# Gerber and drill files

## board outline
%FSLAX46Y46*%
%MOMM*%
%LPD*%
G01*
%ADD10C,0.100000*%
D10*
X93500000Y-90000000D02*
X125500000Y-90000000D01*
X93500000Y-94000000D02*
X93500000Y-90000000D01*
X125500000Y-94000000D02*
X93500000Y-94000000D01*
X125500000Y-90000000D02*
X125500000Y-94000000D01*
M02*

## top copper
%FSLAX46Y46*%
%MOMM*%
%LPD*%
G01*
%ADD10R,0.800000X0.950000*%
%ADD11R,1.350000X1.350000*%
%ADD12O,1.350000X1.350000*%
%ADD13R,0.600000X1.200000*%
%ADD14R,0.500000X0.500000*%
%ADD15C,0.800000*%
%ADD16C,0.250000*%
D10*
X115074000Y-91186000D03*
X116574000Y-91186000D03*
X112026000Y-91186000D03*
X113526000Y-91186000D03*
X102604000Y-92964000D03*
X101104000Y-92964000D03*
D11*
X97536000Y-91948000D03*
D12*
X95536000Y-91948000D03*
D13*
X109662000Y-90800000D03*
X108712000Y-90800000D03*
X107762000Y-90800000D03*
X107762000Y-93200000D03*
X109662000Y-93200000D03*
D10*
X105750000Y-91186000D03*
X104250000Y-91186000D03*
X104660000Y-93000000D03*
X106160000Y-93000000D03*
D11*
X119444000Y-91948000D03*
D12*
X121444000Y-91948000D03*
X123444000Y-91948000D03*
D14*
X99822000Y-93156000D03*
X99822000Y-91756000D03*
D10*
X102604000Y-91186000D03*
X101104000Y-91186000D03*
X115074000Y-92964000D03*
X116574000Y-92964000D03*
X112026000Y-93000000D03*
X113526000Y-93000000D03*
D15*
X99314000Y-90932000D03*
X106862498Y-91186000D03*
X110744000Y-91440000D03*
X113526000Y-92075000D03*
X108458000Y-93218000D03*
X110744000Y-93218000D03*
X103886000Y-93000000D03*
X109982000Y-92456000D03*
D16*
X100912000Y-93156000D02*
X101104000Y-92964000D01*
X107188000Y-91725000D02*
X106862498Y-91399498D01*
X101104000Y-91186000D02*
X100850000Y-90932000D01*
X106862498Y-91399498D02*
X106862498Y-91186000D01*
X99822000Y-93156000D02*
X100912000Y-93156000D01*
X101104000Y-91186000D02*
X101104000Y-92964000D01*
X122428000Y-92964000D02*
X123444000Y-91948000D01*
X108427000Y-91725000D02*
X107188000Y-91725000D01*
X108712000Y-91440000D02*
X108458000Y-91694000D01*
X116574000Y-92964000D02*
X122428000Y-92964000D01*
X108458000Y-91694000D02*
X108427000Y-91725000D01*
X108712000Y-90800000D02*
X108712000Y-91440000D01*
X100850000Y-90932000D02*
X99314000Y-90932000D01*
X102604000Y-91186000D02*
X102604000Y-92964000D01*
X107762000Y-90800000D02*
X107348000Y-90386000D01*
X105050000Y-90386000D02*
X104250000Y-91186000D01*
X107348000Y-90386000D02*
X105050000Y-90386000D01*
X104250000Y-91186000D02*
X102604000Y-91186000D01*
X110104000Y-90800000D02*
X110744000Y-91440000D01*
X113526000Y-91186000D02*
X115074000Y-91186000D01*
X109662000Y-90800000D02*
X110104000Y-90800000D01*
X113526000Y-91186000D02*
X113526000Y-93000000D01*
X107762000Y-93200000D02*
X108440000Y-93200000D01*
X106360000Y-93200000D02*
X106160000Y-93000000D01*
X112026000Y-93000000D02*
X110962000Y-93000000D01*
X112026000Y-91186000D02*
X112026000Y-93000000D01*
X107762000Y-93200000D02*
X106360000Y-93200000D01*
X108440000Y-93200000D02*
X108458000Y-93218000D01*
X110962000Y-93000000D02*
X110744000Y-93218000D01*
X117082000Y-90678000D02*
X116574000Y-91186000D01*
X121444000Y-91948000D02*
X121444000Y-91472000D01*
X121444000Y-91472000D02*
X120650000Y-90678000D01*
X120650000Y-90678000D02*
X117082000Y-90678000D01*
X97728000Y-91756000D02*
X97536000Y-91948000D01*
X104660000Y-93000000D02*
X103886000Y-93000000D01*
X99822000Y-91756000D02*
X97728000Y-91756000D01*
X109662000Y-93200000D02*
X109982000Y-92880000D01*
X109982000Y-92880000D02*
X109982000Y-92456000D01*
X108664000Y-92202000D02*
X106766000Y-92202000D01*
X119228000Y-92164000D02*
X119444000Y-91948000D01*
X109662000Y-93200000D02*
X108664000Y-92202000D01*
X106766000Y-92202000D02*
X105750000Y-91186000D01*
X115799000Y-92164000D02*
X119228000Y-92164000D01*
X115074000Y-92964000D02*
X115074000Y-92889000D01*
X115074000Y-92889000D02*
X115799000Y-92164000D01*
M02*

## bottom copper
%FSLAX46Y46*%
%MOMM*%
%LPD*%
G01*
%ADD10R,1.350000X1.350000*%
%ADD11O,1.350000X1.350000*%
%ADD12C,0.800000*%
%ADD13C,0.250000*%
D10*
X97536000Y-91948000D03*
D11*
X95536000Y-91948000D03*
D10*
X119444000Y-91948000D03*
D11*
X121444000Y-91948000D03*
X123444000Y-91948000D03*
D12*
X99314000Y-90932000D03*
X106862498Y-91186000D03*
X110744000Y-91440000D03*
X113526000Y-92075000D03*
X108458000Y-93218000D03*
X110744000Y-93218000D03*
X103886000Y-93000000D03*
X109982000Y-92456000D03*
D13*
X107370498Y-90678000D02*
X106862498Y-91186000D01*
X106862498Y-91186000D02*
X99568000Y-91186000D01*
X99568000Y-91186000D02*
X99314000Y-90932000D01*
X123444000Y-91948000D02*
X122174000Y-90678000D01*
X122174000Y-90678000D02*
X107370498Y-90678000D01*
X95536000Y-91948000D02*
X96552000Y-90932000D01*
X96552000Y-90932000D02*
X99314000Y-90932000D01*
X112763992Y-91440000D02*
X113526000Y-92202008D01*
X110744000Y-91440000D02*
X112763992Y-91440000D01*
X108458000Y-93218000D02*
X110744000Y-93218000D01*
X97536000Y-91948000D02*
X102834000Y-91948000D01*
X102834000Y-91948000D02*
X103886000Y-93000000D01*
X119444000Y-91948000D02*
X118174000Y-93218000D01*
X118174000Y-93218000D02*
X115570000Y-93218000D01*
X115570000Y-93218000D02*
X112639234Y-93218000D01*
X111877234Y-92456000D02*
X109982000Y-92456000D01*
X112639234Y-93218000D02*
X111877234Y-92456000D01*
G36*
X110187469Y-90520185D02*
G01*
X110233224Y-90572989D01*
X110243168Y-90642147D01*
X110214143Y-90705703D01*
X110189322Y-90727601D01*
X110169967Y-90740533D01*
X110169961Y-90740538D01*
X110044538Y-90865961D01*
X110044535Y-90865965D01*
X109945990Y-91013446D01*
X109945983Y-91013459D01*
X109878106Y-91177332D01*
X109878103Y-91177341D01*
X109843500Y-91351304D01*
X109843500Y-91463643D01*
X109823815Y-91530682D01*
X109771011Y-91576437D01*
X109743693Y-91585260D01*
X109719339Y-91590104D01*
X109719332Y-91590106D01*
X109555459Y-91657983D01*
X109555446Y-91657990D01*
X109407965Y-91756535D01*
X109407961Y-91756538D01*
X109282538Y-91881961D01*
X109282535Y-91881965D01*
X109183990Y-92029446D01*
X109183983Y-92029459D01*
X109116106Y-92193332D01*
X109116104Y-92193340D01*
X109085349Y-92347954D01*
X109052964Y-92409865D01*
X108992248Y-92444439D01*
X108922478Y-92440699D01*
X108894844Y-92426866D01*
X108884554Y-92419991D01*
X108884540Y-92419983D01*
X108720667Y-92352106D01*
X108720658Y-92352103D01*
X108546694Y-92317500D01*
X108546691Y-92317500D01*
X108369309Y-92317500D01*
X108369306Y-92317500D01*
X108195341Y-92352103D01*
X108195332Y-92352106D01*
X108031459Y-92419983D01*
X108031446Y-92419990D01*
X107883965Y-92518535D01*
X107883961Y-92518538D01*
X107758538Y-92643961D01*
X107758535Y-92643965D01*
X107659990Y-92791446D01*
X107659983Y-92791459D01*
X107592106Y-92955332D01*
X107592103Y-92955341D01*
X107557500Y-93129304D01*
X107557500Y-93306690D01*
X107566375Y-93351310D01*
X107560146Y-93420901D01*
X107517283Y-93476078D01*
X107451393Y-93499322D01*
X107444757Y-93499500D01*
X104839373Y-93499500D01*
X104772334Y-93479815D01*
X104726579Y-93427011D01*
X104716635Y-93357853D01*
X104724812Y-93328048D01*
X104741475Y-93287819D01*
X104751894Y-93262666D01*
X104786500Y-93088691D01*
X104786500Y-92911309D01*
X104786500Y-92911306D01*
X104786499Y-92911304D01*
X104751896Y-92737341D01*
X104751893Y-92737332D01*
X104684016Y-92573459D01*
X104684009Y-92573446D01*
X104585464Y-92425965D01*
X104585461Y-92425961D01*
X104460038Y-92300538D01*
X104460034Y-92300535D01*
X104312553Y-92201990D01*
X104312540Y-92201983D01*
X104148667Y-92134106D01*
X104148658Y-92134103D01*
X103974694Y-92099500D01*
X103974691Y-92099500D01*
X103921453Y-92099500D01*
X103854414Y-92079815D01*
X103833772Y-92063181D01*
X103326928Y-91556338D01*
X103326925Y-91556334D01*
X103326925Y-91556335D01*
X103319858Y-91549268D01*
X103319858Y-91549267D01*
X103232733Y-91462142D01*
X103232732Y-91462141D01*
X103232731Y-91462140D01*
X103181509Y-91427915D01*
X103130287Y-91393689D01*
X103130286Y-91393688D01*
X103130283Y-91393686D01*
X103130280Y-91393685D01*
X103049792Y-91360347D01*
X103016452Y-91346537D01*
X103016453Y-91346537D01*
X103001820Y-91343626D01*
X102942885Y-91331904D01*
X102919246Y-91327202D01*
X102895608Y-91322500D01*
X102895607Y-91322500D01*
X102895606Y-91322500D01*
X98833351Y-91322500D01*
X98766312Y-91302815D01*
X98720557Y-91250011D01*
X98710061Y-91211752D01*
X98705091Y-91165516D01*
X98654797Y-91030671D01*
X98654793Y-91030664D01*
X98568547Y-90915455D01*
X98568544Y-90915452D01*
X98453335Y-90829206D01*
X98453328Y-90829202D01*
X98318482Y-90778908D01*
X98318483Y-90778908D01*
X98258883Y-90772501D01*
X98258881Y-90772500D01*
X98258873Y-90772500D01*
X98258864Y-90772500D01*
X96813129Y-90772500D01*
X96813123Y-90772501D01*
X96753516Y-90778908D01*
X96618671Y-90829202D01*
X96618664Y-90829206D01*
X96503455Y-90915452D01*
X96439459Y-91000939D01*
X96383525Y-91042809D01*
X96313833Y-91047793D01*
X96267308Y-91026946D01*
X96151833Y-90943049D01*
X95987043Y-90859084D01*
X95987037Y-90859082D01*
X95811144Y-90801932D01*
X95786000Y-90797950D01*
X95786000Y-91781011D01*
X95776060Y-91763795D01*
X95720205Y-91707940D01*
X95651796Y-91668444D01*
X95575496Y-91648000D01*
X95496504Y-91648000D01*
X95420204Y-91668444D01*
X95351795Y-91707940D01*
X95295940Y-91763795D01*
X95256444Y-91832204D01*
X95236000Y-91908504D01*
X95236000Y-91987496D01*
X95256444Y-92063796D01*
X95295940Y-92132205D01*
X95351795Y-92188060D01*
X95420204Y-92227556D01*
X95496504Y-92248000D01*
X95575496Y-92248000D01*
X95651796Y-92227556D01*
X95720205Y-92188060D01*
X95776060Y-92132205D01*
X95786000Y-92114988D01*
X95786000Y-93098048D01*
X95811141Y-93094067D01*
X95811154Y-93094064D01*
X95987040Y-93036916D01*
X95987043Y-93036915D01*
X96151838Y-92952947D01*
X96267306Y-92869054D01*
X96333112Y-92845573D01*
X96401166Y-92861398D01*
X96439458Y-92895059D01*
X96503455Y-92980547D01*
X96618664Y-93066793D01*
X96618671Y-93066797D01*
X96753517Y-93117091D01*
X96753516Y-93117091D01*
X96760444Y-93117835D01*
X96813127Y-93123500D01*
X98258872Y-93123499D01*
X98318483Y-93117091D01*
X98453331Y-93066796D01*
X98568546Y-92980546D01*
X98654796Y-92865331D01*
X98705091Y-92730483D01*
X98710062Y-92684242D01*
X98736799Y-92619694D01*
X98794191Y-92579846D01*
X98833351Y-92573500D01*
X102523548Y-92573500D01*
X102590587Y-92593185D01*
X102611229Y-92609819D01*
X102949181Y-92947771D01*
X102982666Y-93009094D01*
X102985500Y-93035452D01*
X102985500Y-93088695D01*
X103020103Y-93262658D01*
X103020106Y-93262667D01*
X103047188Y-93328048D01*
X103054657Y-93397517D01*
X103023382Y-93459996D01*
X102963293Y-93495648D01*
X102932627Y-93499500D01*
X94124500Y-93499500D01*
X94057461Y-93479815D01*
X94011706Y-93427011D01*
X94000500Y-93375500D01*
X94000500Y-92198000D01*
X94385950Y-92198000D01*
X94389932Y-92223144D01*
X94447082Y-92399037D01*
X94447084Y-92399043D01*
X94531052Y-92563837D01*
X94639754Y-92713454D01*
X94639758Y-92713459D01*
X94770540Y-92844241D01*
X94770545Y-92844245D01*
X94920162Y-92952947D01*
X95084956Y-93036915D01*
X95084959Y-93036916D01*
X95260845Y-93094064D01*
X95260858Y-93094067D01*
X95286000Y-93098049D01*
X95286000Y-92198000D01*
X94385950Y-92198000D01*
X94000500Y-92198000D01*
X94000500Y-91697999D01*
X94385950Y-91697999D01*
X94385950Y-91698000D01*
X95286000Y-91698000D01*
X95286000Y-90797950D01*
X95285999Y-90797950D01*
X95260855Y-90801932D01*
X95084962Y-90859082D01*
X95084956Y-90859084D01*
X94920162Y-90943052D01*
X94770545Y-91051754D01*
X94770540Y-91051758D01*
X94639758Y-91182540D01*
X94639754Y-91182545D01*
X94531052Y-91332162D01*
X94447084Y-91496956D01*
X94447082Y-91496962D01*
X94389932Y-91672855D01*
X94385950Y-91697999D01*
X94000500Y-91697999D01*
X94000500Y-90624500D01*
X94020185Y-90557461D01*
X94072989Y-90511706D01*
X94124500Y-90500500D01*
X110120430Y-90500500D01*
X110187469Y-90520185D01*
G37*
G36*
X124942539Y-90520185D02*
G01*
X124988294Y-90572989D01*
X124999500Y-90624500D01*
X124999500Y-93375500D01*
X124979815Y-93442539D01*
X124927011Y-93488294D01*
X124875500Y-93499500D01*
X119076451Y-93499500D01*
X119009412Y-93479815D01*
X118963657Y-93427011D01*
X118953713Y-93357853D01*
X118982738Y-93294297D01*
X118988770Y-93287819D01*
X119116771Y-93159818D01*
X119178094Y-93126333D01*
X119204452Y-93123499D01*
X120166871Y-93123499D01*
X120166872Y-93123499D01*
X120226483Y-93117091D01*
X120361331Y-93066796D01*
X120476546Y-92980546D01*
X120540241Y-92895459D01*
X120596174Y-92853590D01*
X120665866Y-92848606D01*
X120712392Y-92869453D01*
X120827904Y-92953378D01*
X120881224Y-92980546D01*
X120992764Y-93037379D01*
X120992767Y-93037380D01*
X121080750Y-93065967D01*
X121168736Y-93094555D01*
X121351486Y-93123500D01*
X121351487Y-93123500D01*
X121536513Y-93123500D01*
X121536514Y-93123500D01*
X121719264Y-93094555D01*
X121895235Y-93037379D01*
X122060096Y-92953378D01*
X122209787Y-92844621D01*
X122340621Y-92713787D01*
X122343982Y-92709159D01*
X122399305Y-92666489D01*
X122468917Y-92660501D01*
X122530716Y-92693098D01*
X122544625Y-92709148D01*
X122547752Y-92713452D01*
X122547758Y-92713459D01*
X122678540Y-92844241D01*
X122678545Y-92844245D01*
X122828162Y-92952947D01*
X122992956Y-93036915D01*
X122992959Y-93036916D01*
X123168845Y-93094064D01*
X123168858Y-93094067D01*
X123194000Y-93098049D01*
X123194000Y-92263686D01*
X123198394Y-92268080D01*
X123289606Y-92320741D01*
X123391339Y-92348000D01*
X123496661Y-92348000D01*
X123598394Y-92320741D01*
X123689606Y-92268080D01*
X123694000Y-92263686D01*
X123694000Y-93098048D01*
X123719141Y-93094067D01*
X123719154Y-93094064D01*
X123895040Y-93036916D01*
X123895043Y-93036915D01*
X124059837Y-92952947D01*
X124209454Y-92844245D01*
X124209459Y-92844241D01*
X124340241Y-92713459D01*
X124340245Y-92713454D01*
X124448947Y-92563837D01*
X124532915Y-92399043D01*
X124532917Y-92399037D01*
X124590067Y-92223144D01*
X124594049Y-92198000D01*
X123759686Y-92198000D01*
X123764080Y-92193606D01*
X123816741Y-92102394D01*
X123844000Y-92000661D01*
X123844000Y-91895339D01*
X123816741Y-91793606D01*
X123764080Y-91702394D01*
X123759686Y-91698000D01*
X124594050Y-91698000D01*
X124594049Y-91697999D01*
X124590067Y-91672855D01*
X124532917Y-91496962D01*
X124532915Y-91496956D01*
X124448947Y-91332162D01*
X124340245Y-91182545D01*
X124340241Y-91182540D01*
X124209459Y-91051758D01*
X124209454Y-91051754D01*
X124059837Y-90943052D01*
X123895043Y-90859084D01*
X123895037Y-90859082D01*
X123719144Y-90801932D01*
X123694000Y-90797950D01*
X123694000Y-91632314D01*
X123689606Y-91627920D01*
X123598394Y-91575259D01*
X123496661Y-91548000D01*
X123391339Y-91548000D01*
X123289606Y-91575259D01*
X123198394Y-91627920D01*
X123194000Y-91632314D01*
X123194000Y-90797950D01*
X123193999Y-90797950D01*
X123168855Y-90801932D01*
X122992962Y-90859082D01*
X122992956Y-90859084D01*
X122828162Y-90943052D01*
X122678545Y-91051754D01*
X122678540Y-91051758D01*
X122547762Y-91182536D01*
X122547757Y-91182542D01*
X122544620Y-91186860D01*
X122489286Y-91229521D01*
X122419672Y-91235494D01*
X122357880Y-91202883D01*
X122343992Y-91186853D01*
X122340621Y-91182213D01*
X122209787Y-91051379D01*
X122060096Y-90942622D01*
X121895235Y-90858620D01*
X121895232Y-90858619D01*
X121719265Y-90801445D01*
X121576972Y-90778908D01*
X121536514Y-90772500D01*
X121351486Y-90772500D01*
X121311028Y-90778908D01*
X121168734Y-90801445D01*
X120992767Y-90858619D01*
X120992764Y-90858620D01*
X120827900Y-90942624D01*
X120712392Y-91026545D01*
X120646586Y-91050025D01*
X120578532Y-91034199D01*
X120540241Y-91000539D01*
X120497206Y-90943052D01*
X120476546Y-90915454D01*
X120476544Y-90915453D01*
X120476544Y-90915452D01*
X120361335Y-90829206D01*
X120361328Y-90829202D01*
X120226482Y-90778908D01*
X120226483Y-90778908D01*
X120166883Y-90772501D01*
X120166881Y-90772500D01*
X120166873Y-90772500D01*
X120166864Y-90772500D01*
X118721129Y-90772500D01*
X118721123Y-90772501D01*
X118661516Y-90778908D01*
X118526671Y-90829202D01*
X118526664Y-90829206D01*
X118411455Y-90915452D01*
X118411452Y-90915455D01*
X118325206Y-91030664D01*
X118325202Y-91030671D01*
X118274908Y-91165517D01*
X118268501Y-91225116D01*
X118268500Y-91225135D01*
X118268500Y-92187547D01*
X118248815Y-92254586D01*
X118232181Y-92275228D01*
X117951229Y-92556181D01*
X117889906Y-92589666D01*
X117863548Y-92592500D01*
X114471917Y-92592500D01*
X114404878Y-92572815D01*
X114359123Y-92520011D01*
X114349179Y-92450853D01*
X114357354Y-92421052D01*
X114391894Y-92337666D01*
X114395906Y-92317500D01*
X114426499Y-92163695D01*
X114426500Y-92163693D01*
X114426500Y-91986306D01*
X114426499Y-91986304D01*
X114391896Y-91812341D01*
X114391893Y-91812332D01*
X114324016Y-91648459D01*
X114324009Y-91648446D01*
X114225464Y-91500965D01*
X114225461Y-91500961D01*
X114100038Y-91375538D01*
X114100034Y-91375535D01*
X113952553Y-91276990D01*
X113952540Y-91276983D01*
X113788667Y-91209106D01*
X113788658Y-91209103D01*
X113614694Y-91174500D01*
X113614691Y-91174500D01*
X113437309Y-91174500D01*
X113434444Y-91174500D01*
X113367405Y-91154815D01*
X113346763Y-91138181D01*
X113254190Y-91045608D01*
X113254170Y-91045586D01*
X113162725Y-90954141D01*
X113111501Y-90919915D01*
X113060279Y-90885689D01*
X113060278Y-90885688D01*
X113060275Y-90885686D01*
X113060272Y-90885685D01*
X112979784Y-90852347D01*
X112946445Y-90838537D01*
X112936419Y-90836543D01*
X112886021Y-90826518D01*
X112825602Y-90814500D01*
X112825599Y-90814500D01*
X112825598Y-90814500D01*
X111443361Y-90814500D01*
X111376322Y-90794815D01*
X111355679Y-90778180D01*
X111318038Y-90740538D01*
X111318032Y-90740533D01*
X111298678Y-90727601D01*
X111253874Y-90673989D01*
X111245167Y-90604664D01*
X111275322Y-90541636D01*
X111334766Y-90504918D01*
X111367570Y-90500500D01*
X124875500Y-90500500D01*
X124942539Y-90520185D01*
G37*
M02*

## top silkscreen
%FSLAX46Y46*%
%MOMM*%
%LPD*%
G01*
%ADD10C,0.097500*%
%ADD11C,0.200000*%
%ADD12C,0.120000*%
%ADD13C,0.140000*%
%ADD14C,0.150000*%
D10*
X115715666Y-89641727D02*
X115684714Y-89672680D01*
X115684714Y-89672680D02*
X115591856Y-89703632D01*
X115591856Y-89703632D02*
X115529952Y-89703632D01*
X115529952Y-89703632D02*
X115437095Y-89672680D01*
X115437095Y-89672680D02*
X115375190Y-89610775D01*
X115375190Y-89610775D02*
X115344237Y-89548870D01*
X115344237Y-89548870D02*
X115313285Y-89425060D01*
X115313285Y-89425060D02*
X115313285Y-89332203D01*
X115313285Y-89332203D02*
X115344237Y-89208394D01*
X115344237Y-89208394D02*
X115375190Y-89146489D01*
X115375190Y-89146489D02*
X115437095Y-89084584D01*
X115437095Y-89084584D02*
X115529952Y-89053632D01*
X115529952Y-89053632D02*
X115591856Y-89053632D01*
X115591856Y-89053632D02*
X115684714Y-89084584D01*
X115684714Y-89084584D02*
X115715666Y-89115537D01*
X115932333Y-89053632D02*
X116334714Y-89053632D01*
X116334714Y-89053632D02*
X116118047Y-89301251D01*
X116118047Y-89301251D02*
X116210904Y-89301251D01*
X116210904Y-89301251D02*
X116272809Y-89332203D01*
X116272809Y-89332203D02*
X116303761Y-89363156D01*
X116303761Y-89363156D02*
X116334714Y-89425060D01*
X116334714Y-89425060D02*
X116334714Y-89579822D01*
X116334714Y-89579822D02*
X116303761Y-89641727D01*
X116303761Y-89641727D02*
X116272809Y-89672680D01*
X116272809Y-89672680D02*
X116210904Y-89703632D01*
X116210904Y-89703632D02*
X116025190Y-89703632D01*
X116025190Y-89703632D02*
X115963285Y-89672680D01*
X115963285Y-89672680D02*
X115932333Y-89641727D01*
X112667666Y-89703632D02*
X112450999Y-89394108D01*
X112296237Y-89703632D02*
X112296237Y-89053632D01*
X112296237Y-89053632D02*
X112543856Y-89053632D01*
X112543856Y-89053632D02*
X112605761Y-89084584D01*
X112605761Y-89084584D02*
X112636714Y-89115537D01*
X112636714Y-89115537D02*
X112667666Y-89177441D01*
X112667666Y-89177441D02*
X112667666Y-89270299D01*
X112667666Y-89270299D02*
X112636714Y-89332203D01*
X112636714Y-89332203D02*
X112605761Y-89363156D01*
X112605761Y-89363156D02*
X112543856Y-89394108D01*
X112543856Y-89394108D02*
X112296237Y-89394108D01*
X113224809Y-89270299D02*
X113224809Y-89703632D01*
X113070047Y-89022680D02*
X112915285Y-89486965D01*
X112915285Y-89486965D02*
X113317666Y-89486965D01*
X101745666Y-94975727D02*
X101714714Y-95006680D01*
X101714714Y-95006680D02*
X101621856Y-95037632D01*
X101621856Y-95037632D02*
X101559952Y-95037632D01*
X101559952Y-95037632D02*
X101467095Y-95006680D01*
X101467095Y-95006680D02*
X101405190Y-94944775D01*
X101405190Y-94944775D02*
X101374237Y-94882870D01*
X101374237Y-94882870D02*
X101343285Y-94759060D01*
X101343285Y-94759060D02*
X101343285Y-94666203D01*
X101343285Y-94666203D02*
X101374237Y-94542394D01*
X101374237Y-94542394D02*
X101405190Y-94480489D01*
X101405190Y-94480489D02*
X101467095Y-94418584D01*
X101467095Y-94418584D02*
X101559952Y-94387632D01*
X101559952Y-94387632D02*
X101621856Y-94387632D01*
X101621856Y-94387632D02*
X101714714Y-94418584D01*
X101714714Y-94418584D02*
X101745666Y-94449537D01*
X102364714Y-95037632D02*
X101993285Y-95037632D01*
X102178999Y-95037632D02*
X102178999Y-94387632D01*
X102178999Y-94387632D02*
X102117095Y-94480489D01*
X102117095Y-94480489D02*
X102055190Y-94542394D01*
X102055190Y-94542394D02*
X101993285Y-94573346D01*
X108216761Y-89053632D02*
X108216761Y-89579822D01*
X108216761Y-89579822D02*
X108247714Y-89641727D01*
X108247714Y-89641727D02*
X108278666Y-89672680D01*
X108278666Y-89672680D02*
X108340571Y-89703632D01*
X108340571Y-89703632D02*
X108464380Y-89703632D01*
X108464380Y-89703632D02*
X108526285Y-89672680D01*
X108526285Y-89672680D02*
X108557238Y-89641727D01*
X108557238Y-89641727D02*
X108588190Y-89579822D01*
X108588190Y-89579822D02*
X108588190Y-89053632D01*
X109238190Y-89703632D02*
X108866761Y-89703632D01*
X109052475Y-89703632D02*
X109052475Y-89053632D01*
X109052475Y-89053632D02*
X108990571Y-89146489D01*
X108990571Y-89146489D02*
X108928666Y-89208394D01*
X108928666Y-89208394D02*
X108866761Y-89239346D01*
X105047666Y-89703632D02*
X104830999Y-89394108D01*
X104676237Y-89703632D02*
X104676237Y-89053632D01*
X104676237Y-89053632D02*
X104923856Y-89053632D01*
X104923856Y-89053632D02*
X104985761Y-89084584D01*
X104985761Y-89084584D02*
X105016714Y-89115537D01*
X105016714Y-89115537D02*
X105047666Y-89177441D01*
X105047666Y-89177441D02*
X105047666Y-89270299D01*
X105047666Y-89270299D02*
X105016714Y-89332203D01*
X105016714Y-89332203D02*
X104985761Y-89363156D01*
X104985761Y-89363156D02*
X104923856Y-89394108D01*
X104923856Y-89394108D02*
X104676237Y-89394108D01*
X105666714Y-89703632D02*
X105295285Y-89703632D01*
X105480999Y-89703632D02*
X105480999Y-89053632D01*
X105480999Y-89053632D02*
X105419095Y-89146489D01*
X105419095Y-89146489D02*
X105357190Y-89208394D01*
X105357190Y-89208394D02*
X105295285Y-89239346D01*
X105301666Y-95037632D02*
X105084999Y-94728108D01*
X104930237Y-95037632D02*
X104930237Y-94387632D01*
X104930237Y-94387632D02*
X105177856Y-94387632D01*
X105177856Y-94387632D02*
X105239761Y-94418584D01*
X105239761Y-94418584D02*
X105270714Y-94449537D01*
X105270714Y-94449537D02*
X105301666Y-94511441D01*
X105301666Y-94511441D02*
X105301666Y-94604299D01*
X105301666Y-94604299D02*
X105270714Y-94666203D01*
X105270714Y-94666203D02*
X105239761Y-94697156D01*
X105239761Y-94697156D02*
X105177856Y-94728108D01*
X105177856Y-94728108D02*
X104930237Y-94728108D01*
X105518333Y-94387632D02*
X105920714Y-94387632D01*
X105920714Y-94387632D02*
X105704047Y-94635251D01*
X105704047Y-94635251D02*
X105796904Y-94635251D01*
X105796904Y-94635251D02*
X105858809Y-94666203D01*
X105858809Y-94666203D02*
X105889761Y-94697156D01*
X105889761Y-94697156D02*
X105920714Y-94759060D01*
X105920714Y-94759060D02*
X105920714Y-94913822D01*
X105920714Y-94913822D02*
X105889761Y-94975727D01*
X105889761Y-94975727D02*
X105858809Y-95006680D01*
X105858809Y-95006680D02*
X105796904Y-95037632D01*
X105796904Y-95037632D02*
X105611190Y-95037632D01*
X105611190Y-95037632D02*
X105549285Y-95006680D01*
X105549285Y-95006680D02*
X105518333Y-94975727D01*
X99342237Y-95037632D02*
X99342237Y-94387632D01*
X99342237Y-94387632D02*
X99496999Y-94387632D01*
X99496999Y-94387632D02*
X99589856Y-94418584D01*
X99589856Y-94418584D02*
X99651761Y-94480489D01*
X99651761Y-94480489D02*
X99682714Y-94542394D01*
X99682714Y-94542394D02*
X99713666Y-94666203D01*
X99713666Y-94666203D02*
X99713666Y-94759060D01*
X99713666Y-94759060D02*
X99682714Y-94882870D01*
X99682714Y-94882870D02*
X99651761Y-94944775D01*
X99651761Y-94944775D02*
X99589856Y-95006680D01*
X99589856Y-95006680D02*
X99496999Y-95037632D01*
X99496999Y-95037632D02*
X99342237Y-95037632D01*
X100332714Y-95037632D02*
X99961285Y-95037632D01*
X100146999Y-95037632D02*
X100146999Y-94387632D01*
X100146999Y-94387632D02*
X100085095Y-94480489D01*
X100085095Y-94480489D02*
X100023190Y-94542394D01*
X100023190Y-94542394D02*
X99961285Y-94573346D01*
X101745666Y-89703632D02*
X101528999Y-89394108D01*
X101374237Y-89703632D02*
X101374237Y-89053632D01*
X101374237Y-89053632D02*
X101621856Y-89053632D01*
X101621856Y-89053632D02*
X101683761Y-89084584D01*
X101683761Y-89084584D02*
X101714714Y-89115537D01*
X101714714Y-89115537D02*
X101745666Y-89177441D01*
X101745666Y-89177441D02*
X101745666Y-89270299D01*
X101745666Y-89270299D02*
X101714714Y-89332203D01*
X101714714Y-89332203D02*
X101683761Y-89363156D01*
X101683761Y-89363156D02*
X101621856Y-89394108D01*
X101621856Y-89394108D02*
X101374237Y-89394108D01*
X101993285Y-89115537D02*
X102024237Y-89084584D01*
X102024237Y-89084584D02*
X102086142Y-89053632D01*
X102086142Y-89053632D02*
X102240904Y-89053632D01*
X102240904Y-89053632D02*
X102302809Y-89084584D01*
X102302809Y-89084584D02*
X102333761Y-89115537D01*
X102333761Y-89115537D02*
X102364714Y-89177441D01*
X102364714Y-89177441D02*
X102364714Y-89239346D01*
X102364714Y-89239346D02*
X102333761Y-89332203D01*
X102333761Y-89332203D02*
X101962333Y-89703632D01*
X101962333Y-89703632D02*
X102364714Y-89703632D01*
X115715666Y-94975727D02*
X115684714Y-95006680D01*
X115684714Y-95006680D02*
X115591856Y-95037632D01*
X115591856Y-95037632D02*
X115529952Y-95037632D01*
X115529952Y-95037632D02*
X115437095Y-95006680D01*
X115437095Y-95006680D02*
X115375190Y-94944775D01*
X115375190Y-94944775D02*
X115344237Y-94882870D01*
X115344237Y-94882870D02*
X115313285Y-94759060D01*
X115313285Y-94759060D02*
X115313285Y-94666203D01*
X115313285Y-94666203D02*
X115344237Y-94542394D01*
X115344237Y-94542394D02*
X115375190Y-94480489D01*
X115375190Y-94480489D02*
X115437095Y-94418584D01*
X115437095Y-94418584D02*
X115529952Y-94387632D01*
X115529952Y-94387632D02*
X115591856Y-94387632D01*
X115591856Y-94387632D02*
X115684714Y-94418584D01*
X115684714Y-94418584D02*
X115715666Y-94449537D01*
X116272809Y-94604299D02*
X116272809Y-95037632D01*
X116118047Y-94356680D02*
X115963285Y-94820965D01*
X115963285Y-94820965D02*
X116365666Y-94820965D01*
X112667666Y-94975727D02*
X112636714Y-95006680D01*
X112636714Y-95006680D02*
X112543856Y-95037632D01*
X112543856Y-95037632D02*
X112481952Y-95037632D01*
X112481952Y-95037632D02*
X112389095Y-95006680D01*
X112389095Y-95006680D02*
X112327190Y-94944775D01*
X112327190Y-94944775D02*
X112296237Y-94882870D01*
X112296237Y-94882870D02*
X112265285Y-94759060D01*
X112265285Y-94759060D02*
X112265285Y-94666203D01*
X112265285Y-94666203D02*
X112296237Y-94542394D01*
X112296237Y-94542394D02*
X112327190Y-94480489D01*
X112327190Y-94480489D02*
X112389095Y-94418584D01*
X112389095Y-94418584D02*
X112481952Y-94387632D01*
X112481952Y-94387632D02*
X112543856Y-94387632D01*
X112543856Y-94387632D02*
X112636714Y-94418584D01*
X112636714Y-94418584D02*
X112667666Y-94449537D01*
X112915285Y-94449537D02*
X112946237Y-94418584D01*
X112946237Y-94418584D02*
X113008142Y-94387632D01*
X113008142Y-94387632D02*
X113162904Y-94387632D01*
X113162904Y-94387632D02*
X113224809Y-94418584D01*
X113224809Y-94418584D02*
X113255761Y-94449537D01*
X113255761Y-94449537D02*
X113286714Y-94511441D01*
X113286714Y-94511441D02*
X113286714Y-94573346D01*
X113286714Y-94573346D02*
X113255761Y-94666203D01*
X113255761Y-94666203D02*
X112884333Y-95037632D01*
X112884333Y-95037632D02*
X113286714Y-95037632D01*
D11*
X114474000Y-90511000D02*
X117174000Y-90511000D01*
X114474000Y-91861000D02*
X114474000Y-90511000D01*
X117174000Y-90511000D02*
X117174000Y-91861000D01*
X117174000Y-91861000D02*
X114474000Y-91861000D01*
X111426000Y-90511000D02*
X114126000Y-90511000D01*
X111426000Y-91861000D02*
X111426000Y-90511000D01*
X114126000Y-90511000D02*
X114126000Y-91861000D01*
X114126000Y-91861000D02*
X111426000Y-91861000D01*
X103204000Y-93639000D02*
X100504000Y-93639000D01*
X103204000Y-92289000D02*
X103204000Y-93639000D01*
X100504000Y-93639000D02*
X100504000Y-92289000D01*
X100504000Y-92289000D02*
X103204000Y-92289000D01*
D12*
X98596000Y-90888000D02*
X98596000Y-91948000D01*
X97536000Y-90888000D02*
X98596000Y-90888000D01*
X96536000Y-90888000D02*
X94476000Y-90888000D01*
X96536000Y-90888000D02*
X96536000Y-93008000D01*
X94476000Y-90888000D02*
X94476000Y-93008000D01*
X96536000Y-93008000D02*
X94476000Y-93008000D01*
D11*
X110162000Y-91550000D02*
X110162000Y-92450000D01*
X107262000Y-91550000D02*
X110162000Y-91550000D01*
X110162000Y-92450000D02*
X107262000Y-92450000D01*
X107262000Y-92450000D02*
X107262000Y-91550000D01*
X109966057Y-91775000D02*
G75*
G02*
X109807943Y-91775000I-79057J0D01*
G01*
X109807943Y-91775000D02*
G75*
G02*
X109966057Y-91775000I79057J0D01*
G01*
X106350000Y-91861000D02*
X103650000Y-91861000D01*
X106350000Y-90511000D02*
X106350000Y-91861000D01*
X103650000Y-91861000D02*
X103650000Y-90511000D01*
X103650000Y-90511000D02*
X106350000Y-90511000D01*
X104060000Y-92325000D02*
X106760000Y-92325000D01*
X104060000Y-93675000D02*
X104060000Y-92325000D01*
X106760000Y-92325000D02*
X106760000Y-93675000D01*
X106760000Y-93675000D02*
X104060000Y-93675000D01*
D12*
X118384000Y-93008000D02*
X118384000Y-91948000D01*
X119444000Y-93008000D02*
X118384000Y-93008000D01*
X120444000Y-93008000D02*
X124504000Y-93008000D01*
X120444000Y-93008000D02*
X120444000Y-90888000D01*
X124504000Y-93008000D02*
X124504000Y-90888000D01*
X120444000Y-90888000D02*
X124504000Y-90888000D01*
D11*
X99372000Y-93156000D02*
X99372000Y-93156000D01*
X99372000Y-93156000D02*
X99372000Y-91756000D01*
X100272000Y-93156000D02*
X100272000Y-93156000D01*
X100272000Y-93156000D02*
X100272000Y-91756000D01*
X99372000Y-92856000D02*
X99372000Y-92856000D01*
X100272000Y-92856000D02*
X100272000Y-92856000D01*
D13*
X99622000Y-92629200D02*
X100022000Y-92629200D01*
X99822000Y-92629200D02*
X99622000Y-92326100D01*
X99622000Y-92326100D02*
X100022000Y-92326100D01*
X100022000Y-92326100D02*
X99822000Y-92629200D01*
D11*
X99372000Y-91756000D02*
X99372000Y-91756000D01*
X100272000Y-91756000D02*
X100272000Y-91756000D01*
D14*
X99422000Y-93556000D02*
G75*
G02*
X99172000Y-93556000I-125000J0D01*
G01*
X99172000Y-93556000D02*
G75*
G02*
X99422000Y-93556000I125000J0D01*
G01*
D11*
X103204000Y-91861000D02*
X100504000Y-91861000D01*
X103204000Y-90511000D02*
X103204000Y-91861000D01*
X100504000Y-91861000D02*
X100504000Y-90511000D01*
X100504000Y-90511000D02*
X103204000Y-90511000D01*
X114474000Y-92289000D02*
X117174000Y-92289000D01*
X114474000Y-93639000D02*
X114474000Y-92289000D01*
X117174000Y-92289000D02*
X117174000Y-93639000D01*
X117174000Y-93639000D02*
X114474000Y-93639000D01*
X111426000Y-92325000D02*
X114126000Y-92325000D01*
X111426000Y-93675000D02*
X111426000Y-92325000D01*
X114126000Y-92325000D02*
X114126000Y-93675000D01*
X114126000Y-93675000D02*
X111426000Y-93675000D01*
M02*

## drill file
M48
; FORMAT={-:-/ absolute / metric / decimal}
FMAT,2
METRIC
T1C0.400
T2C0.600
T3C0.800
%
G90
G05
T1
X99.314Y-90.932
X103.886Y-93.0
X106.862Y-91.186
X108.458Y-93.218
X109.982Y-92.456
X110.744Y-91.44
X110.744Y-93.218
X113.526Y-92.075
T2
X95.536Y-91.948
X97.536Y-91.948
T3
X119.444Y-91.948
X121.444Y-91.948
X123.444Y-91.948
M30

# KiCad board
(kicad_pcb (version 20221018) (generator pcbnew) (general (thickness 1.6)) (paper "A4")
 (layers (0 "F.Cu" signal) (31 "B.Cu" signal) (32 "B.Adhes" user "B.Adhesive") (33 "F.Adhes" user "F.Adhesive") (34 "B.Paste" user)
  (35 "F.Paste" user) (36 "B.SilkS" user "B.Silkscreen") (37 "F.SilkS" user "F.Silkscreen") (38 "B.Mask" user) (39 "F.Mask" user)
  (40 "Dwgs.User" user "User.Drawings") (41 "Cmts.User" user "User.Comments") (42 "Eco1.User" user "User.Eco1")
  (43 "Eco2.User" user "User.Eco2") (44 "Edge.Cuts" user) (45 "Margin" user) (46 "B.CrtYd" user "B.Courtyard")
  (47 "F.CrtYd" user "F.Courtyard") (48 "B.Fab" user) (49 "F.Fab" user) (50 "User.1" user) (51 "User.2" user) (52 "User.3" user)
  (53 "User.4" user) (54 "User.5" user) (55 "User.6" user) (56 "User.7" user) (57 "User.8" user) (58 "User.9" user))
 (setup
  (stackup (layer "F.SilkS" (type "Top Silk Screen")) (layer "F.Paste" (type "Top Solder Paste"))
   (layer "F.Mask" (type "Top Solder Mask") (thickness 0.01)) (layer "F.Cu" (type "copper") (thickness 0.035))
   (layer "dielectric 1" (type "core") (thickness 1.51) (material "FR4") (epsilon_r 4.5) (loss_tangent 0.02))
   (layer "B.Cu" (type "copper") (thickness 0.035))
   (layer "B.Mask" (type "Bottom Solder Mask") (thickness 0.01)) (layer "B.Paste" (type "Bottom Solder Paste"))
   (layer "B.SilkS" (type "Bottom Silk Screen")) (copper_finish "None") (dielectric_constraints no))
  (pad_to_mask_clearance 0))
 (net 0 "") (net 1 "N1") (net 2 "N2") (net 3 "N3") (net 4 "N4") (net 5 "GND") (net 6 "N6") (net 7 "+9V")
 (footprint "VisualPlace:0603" (layer "F.Cu") (at 115.824 91.186)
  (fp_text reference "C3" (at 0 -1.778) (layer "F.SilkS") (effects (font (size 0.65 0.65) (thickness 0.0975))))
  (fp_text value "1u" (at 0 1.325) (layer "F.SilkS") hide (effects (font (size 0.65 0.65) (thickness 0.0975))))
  (fp_line (start -1.35 -0.675) (end 1.35 -0.675) (stroke (width 0.2) (type solid)) (layer "F.SilkS"))
  (fp_line (start -1.35 0.675) (end -1.35 -0.675) (stroke (width 0.2) (type solid)) (layer "F.SilkS"))
  (fp_line (start 1.35 -0.675) (end 1.35 0.675) (stroke (width 0.2) (type solid)) (layer "F.SilkS"))
  (fp_line (start 1.35 0.675) (end -1.35 0.675) (stroke (width 0.2) (type solid)) (layer "F.SilkS"))
  (pad "1" smd rect (at -0.75 0) (size 0.8 0.95) (layers "F.Cu" "F.Paste" "F.Mask") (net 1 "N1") (thermal_bridge_angle 45))
  (pad "2" smd rect (at 0.75 0) (size 0.8 0.95) (layers "F.Cu" "F.Paste" "F.Mask") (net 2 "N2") (thermal_bridge_angle 45)))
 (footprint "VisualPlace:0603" (layer "F.Cu") (at 112.776 91.186)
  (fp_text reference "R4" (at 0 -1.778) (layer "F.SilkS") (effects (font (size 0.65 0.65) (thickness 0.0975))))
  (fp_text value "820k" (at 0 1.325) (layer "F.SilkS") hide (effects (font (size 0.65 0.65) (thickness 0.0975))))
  (fp_line (start -1.35 -0.675) (end 1.35 -0.675) (stroke (width 0.2) (type solid)) (layer "F.SilkS"))
  (fp_line (start -1.35 0.675) (end -1.35 -0.675) (stroke (width 0.2) (type solid)) (layer "F.SilkS"))
  (fp_line (start 1.35 -0.675) (end 1.35 0.675) (stroke (width 0.2) (type solid)) (layer "F.SilkS"))
  (fp_line (start 1.35 0.675) (end -1.35 0.675) (stroke (width 0.2) (type solid)) (layer "F.SilkS"))
  (pad "1" smd rect (at -0.75 0) (size 0.8 0.95) (layers "F.Cu" "F.Paste" "F.Mask") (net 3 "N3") (thermal_bridge_angle 45))
  (pad "2" smd rect (at 0.75 0) (size 0.8 0.95) (layers "F.Cu" "F.Paste" "F.Mask") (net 1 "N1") (thermal_bridge_angle 45)))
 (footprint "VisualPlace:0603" (layer "F.Cu") (at 101.854 92.964 180)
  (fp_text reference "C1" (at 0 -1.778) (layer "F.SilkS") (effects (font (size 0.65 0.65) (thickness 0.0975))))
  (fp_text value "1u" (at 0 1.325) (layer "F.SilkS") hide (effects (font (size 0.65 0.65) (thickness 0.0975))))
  (fp_line (start -1.35 -0.675) (end 1.35 -0.675) (stroke (width 0.2) (type solid)) (layer "F.SilkS"))
  (fp_line (start -1.35 0.675) (end -1.35 -0.675) (stroke (width 0.2) (type solid)) (layer "F.SilkS"))
  (fp_line (start 1.35 -0.675) (end 1.35 0.675) (stroke (width 0.2) (type solid)) (layer "F.SilkS"))
  (fp_line (start 1.35 0.675) (end -1.35 0.675) (stroke (width 0.2) (type solid)) (layer "F.SilkS"))
  (pad "1" smd rect (at -0.75 0 180) (size 0.8 0.95) (layers "F.Cu" "F.Paste" "F.Mask") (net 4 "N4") (thermal_bridge_angle 45))
  (pad "2" smd rect (at 0.75 0 180) (size 0.8 0.95) (layers "F.Cu" "F.Paste" "F.Mask") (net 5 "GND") (thermal_bridge_angle 45)))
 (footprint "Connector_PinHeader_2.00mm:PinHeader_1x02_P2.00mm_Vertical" (layer "F.Cu") (at 97.536 91.948 -90)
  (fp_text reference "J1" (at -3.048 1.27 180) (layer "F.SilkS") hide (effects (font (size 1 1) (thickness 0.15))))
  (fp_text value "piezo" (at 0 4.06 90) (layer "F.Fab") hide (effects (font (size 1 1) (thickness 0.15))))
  (fp_line (start -1.06 -1.06) (end 0 -1.06) (stroke (width 0.12) (type solid)) (layer "F.SilkS"))
  (fp_line (start -1.06 0) (end -1.06 -1.06) (stroke (width 0.12) (type solid)) (layer "F.SilkS"))
  (fp_line (start -1.06 1) (end -1.06 3.06) (stroke (width 0.12) (type solid)) (layer "F.SilkS"))
  (fp_line (start -1.06 1) (end 1.06 1) (stroke (width 0.12) (type solid)) (layer "F.SilkS"))
  (fp_line (start -1.06 3.06) (end 1.06 3.06) (stroke (width 0.12) (type solid)) (layer "F.SilkS"))
  (fp_line (start 1.06 1) (end 1.06 3.06) (stroke (width 0.12) (type solid)) (layer "F.SilkS"))
  (pad "1" thru_hole rect (at 0 0 270) (size 1.35 1.35) (drill 0.6) (layers "*.Cu" "*.Mask") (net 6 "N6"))
  (pad "2" thru_hole oval (at 0 2 270) (size 1.35 1.35) (drill 0.6) (layers "*.Cu" "*.Mask") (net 5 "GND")))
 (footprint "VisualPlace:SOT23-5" (layer "F.Cu") (at 108.712 92 -90)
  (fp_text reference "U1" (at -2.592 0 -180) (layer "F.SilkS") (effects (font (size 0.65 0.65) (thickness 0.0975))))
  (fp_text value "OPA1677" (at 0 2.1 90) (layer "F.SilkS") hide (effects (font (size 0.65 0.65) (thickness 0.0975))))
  (fp_line (start -0.45 -1.45) (end 0.45 -1.45) (stroke (width 0.2) (type solid)) (layer "F.SilkS"))
  (fp_line (start -0.45 1.45) (end -0.45 -1.45) (stroke (width 0.2) (type solid)) (layer "F.SilkS"))
  (fp_line (start 0.45 -1.45) (end 0.45 1.45) (stroke (width 0.2) (type solid)) (layer "F.SilkS"))
  (fp_line (start 0.45 1.45) (end -0.45 1.45) (stroke (width 0.2) (type solid)) (layer "F.SilkS"))
  (fp_circle (center -0.225 -1.175) (end -0.3 -1.15) (stroke (width 0.2) (type solid)) (fill none) (layer "F.SilkS"))
  (pad "1" smd rect (at -1.2 -0.95 270) (size 1.2 0.6) (layers "F.Cu" "F.Paste" "F.Mask") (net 1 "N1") (thermal_bridge_angle 45))
  (pad "2" smd rect (at -1.2 0 270) (size 1.2 0.6) (layers "F.Cu" "F.Paste" "F.Mask") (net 5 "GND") (thermal_bridge_angle 45))
  (pad "3" smd rect (at -1.2 0.95 270) (size 1.2 0.6) (layers "F.Cu" "F.Paste" "F.Mask") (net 4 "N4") (thermal_bridge_angle 45))
  (pad "4" smd rect (at 1.2 0.95 270) (size 1.2 0.6) (layers "F.Cu" "F.Paste" "F.Mask") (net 3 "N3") (thermal_bridge_angle 45))
  (pad "5" smd rect (at 1.2 -0.95 270) (size 1.2 0.6) (layers "F.Cu" "F.Paste" "F.Mask") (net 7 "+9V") (thermal_bridge_angle 45)))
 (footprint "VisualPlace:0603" (layer "F.Cu") (at 105 91.186 180)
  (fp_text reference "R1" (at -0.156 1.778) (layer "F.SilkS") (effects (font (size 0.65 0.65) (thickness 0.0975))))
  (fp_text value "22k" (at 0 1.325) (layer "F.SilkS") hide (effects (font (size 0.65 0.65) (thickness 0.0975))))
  (fp_line (start -1.35 -0.675) (end 1.35 -0.675) (stroke (width 0.2) (type solid)) (layer "F.SilkS"))
  (fp_line (start -1.35 0.675) (end -1.35 -0.675) (stroke (width 0.2) (type solid)) (layer "F.SilkS"))
  (fp_line (start 1.35 -0.675) (end 1.35 0.675) (stroke (width 0.2) (type solid)) (layer "F.SilkS"))
  (fp_line (start 1.35 0.675) (end -1.35 0.675) (stroke (width 0.2) (type solid)) (layer "F.SilkS"))
  (pad "1" smd rect (at -0.75 0 180) (size 0.8 0.95) (layers "F.Cu" "F.Paste" "F.Mask") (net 7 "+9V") (thermal_bridge_angle 45))
  (pad "2" smd rect (at 0.75 0 180) (size 0.8 0.95) (layers "F.Cu" "F.Paste" "F.Mask") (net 4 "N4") (thermal_bridge_angle 45)))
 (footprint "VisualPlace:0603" (layer "F.Cu") (at 105.41 93)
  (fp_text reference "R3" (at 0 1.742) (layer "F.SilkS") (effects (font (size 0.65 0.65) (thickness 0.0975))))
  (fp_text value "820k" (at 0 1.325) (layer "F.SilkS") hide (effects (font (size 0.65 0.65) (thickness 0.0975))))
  (fp_line (start -1.35 -0.675) (end 1.35 -0.675) (stroke (width 0.2) (type solid)) (layer "F.SilkS"))
  (fp_line (start -1.35 0.675) (end -1.35 -0.675) (stroke (width 0.2) (type solid)) (layer "F.SilkS"))
  (fp_line (start 1.35 -0.675) (end 1.35 0.675) (stroke (width 0.2) (type solid)) (layer "F.SilkS"))
  (fp_line (start 1.35 0.675) (end -1.35 0.675) (stroke (width 0.2) (type solid)) (layer "F.SilkS"))
  (pad "1" smd rect (at -0.75 0) (size 0.8 0.95) (layers "F.Cu" "F.Paste" "F.Mask") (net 6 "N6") (thermal_bridge_angle 45))
  (pad "2" smd rect (at 0.75 0) (size 0.8 0.95) (layers "F.Cu" "F.Paste" "F.Mask") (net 3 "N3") (thermal_bridge_angle 45)))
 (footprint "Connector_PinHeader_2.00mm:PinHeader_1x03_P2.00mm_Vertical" (layer "F.Cu") (at 119.444 91.948 90)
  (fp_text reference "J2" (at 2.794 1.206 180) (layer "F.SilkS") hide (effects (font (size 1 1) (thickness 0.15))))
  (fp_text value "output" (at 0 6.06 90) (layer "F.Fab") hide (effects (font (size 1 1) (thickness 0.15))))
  (fp_line (start -1.06 -1.06) (end 0 -1.06) (stroke (width 0.12) (type solid)) (layer "F.SilkS"))
  (fp_line (start -1.06 0) (end -1.06 -1.06) (stroke (width 0.12) (type solid)) (layer "F.SilkS"))
  (fp_line (start -1.06 1) (end -1.06 5.06) (stroke (width 0.12) (type solid)) (layer "F.SilkS"))
  (fp_line (start -1.06 1) (end 1.06 1) (stroke (width 0.12) (type solid)) (layer "F.SilkS"))
  (fp_line (start -1.06 5.06) (end 1.06 5.06) (stroke (width 0.12) (type solid)) (layer "F.SilkS"))
  (fp_line (start 1.06 1) (end 1.06 5.06) (stroke (width 0.12) (type solid)) (layer "F.SilkS"))
  (pad "1" thru_hole rect (at 0 0 90) (size 1.35 1.35) (drill 0.8) (layers "*.Cu" "*.Mask") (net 7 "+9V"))
  (pad "2" thru_hole oval (at 0 2 90) (size 1.35 1.35) (drill 0.8) (layers "*.Cu" "*.Mask") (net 2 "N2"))
  (pad "3" thru_hole oval (at 0 4 90) (size 1.35 1.35) (drill 0.8) (layers "*.Cu" "*.Mask") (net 5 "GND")))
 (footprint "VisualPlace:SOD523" (layer "F.Cu") (at 99.822 92.456 90)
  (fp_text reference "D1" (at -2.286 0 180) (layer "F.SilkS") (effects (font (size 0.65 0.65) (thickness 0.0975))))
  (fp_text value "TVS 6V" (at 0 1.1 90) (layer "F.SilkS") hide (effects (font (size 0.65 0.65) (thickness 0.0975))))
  (fp_line (start -0.7 -0.45) (end -0.7 -0.45) (stroke (width 0.2) (type solid)) (layer "F.SilkS"))
  (fp_line (start -0.7 -0.45) (end 0.7 -0.45) (stroke (width 0.2) (type solid)) (layer "F.SilkS"))
  (fp_line (start -0.7 0.45) (end -0.7 0.45) (stroke (width 0.2) (type solid)) (layer "F.SilkS"))
  (fp_line (start -0.7 0.45) (end 0.7 0.45) (stroke (width 0.2) (type solid)) (layer "F.SilkS"))
  (fp_line (start -0.4 -0.45) (end -0.4 -0.45) (stroke (width 0.2) (type solid)) (layer "F.SilkS"))
  (fp_line (start -0.4 0.45) (end -0.4 0.45) (stroke (width 0.2) (type solid)) (layer "F.SilkS"))
  (fp_line (start -0.1732 -0.2) (end -0.1732 0.2) (stroke (width 0.14) (type solid)) (layer "F.SilkS"))
  (fp_line (start -0.1732 0) (end 0.1299 -0.2) (stroke (width 0.14) (type solid)) (layer "F.SilkS"))
  (fp_line (start 0.1299 -0.2) (end 0.1299 0.2) (stroke (width 0.14) (type solid)) (layer "F.SilkS"))
  (fp_line (start 0.1299 0.2) (end -0.1732 0) (stroke (width 0.14) (type solid)) (layer "F.SilkS"))
  (fp_line (start 0.7 -0.45) (end 0.7 -0.45) (stroke (width 0.2) (type solid)) (layer "F.SilkS"))
  (fp_line (start 0.7 0.45) (end 0.7 0.45) (stroke (width 0.2) (type solid)) (layer "F.SilkS"))
  (fp_circle (center -1.1 -0.525) (end -0.975 -0.525) (stroke (width 0.15) (type solid)) (fill none) (layer "F.SilkS"))
  (pad "1" smd rect (at -0.7 0 90) (size 0.5 0.5) (layers "F.Cu" "F.Paste" "F.Mask") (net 5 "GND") (thermal_bridge_angle 45))
  (pad "2" smd rect (at 0.7 0 90) (size 0.5 0.5) (layers "F.Cu" "F.Paste" "F.Mask") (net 6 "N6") (thermal_bridge_angle 45)))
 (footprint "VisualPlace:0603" (layer "F.Cu") (at 101.854 91.186 180)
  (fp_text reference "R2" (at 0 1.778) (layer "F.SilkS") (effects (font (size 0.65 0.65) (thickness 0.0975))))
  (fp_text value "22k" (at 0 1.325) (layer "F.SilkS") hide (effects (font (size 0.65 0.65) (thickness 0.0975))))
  (fp_line (start -1.35 -0.675) (end 1.35 -0.675) (stroke (width 0.2) (type solid)) (layer "F.SilkS"))
  (fp_line (start -1.35 0.675) (end -1.35 -0.675) (stroke (width 0.2) (type solid)) (layer "F.SilkS"))
  (fp_line (start 1.35 -0.675) (end 1.35 0.675) (stroke (width 0.2) (type solid)) (layer "F.SilkS"))
  (fp_line (start 1.35 0.675) (end -1.35 0.675) (stroke (width 0.2) (type solid)) (layer "F.SilkS"))
  (pad "1" smd rect (at -0.75 0 180) (size 0.8 0.95) (layers "F.Cu" "F.Paste" "F.Mask") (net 4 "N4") (thermal_bridge_angle 45))
  (pad "2" smd rect (at 0.75 0 180) (size 0.8 0.95) (layers "F.Cu" "F.Paste" "F.Mask") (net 5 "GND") (thermal_bridge_angle 45)))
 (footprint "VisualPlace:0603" (layer "F.Cu") (at 115.824 92.964)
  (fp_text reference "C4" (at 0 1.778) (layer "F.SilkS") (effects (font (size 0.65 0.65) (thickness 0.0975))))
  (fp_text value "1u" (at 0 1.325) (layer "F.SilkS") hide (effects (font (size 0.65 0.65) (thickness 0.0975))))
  (fp_line (start -1.35 -0.675) (end 1.35 -0.675) (stroke (width 0.2) (type solid)) (layer "F.SilkS"))
  (fp_line (start -1.35 0.675) (end -1.35 -0.675) (stroke (width 0.2) (type solid)) (layer "F.SilkS"))
  (fp_line (start 1.35 -0.675) (end 1.35 0.675) (stroke (width 0.2) (type solid)) (layer "F.SilkS"))
  (fp_line (start 1.35 0.675) (end -1.35 0.675) (stroke (width 0.2) (type solid)) (layer "F.SilkS"))
  (pad "1" smd rect (at -0.75 0) (size 0.8 0.95) (layers "F.Cu" "F.Paste" "F.Mask") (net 7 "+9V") (thermal_bridge_angle 45))
  (pad "2" smd rect (at 0.75 0) (size 0.8 0.95) (layers "F.Cu" "F.Paste" "F.Mask") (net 5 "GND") (thermal_bridge_angle 45)))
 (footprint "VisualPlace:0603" (layer "F.Cu") (at 112.776 93)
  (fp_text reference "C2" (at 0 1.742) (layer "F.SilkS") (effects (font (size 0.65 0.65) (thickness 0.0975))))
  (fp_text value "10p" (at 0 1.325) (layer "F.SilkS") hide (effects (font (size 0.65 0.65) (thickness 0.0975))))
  (fp_line (start -1.35 -0.675) (end 1.35 -0.675) (stroke (width 0.2) (type solid)) (layer "F.SilkS"))
  (fp_line (start -1.35 0.675) (end -1.35 -0.675) (stroke (width 0.2) (type solid)) (layer "F.SilkS"))
  (fp_line (start 1.35 -0.675) (end 1.35 0.675) (stroke (width 0.2) (type solid)) (layer "F.SilkS"))
  (fp_line (start 1.35 0.675) (end -1.35 0.675) (stroke (width 0.2) (type solid)) (layer "F.SilkS"))
  (pad "1" smd rect (at -0.75 0) (size 0.8 0.95) (layers "F.Cu" "F.Paste" "F.Mask") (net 3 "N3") (thermal_bridge_angle 45))
  (pad "2" smd rect (at 0.75 0) (size 0.8 0.95) (layers "F.Cu" "F.Paste" "F.Mask") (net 1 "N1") (thermal_bridge_angle 45)))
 (gr_line (start 93.5 90) (end 125.5 90) (stroke (width 0.1) (type default)) (layer "Edge.Cuts"))
 (gr_line (start 93.5 94) (end 93.5 90) (stroke (width 0.1) (type default)) (layer "Edge.Cuts"))
 (gr_line (start 125.5 94) (end 93.5 94) (stroke (width 0.1) (type default)) (layer "Edge.Cuts"))
 (gr_line (start 125.5 90) (end 125.5 94) (stroke (width 0.1) (type default)) (layer "Edge.Cuts"))
 (segment (start 100.912 93.156) (end 101.104 92.964) (width 0.25) (layer "F.Cu") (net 5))
 (segment (start 107.188 91.725) (end 106.862498 91.399498) (width 0.25) (layer "F.Cu") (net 5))
 (segment (start 101.104 91.186) (end 100.85 90.932) (width 0.25) (layer "F.Cu") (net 5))
 (segment (start 106.862498 91.399498) (end 106.862498 91.186) (width 0.25) (layer "F.Cu") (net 5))
 (segment (start 99.822 93.156) (end 100.912 93.156) (width 0.25) (layer "F.Cu") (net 5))
 (segment (start 101.104 91.186) (end 101.104 92.964) (width 0.25) (layer "F.Cu") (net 5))
 (segment (start 122.428 92.964) (end 123.444 91.948) (width 0.25) (layer "F.Cu") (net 5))
 (segment (start 108.427 91.725) (end 107.188 91.725) (width 0.25) (layer "F.Cu") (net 5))
 (segment (start 108.712 91.44) (end 108.458 91.694) (width 0.25) (layer "F.Cu") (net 5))
 (segment (start 116.574 92.964) (end 122.428 92.964) (width 0.25) (layer "F.Cu") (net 5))
 (segment (start 108.458 91.694) (end 108.427 91.725) (width 0.25) (layer "F.Cu") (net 5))
 (segment (start 108.712 90.8) (end 108.712 91.44) (width 0.25) (layer "F.Cu") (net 5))
 (segment (start 100.85 90.932) (end 99.314 90.932) (width 0.25) (layer "F.Cu") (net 5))
 (via (at 99.314 90.932) (size 0.8) (drill 0.4) (layers "F.Cu" "B.Cu") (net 5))
 (via (at 106.862498 91.186) (size 0.8) (drill 0.4) (layers "F.Cu" "B.Cu") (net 5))
 (segment (start 107.370498 90.678) (end 106.862498 91.186) (width 0.25) (layer "B.Cu") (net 5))
 (segment (start 106.862498 91.186) (end 99.568 91.186) (width 0.25) (layer "B.Cu") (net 5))
 (segment (start 99.568 91.186) (end 99.314 90.932) (width 0.25) (layer "B.Cu") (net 5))
 (segment (start 123.444 91.948) (end 122.174 90.678) (width 0.25) (layer "B.Cu") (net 5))
 (segment (start 122.174 90.678) (end 107.370498 90.678) (width 0.25) (layer "B.Cu") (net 5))
 (segment (start 95.536 91.948) (end 96.552 90.932) (width 0.25) (layer "B.Cu") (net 5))
 (segment (start 96.552 90.932) (end 99.314 90.932) (width 0.25) (layer "B.Cu") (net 5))
 (segment (start 102.604 91.186) (end 102.604 92.964) (width 0.25) (layer "F.Cu") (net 4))
 (segment (start 107.762 90.8) (end 107.348 90.386) (width 0.25) (layer "F.Cu") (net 4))
 (segment (start 105.05 90.386) (end 104.25 91.186) (width 0.25) (layer "F.Cu") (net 4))
 (segment (start 107.348 90.386) (end 105.05 90.386) (width 0.25) (layer "F.Cu") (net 4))
 (segment (start 104.25 91.186) (end 102.604 91.186) (width 0.25) (layer "F.Cu") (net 4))
 (segment (start 110.104 90.8) (end 110.744 91.44) (width 0.25) (layer "F.Cu") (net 1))
 (segment (start 113.526 91.186) (end 115.074 91.186) (width 0.25) (layer "F.Cu") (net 1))
 (segment (start 109.662 90.8) (end 110.104 90.8) (width 0.25) (layer "F.Cu") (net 1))
 (segment (start 113.526 91.186) (end 113.526 93) (width 0.25) (layer "F.Cu") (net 1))
 (via (at 110.744 91.44) (size 0.8) (drill 0.4) (layers "F.Cu" "B.Cu") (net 1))
 (via (at 113.526 92.075) (size 0.8) (drill 0.4) (layers "F.Cu" "B.Cu") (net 1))
 (segment (start 112.763992 91.44) (end 113.526 92.202008) (width 0.25) (layer "B.Cu") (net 1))
 (segment (start 110.744 91.44) (end 112.763992 91.44) (width 0.25) (layer "B.Cu") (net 1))
 (segment (start 107.762 93.2) (end 108.44 93.2) (width 0.25) (layer "F.Cu") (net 3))
 (segment (start 106.36 93.2) (end 106.16 93) (width 0.25) (layer "F.Cu") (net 3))
 (segment (start 112.026 93) (end 110.962 93) (width 0.25) (layer "F.Cu") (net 3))
 (segment (start 112.026 91.186) (end 112.026 93) (width 0.25) (layer "F.Cu") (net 3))
 (segment (start 107.762 93.2) (end 106.36 93.2) (width 0.25) (layer "F.Cu") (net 3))
 (segment (start 108.44 93.2) (end 108.458 93.218) (width 0.25) (layer "F.Cu") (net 3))
 (segment (start 110.962 93) (end 110.744 93.218) (width 0.25) (layer "F.Cu") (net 3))
 (via (at 108.458 93.218) (size 0.8) (drill 0.4) (layers "F.Cu" "B.Cu") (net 3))
 (via (at 110.744 93.218) (size 0.8) (drill 0.4) (layers "F.Cu" "B.Cu") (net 3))
 (segment (start 108.458 93.218) (end 110.744 93.218) (width 0.25) (layer "B.Cu") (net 3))
 (segment (start 117.082 90.678) (end 116.574 91.186) (width 0.25) (layer "F.Cu") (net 2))
 (segment (start 121.444 91.948) (end 121.444 91.472) (width 0.25) (layer "F.Cu") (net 2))
 (segment (start 121.444 91.472) (end 120.65 90.678) (width 0.25) (layer "F.Cu") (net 2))
 (segment (start 120.65 90.678) (end 117.082 90.678) (width 0.25) (layer "F.Cu") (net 2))
 (segment (start 97.728 91.756) (end 97.536 91.948) (width 0.25) (layer "F.Cu") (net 6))
 (segment (start 104.66 93) (end 103.886 93) (width 0.25) (layer "F.Cu") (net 6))
 (segment (start 99.822 91.756) (end 97.728 91.756) (width 0.25) (layer "F.Cu") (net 6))
 (via (at 103.886 93) (size 0.8) (drill 0.4) (layers "F.Cu" "B.Cu") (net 6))
 (segment (start 97.536 91.948) (end 102.834 91.948) (width 0.25) (layer "B.Cu") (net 6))
 (segment (start 102.834 91.948) (end 103.886 93) (width 0.25) (layer "B.Cu") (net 6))
 (segment (start 109.662 93.2) (end 109.982 92.88) (width 0.25) (layer "F.Cu") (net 7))
 (segment (start 109.982 92.88) (end 109.982 92.456) (width 0.25) (layer "F.Cu") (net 7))
 (segment (start 108.664 92.202) (end 106.766 92.202) (width 0.25) (layer "F.Cu") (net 7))
 (segment (start 119.228 92.164) (end 119.444 91.948) (width 0.25) (layer "F.Cu") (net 7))
 (segment (start 109.662 93.2) (end 108.664 92.202) (width 0.25) (layer "F.Cu") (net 7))
 (segment (start 106.766 92.202) (end 105.75 91.186) (width 0.25) (layer "F.Cu") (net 7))
 (segment (start 115.799 92.164) (end 119.228 92.164) (width 0.25) (layer "F.Cu") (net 7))
 (segment (start 115.074 92.964) (end 115.074 92.889) (width 0.25) (layer "F.Cu") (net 7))
 (segment (start 115.074 92.889) (end 115.799 92.164) (width 0.25) (layer "F.Cu") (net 7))
 (via (at 109.982 92.456) (size 0.8) (drill 0.4) (layers "F.Cu" "B.Cu") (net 7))
 (segment (start 119.444 91.948) (end 118.174 93.218) (width 0.25) (layer "B.Cu") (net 7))
 (segment (start 118.174 93.218) (end 115.57 93.218) (width 0.25) (layer "B.Cu") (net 7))
 (segment (start 115.57 93.218) (end 112.639234 93.218) (width 0.25) (layer "B.Cu") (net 7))
 (segment (start 111.877234 92.456) (end 109.982 92.456) (width 0.25) (layer "B.Cu") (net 7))
 (segment (start 112.639234 93.218) (end 111.877234 92.456) (width 0.25) (layer "B.Cu") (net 7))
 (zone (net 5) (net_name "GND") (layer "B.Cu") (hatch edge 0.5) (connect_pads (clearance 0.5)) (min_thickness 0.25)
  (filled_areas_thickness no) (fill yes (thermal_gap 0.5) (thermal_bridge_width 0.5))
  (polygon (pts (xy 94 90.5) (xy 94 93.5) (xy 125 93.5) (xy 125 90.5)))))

